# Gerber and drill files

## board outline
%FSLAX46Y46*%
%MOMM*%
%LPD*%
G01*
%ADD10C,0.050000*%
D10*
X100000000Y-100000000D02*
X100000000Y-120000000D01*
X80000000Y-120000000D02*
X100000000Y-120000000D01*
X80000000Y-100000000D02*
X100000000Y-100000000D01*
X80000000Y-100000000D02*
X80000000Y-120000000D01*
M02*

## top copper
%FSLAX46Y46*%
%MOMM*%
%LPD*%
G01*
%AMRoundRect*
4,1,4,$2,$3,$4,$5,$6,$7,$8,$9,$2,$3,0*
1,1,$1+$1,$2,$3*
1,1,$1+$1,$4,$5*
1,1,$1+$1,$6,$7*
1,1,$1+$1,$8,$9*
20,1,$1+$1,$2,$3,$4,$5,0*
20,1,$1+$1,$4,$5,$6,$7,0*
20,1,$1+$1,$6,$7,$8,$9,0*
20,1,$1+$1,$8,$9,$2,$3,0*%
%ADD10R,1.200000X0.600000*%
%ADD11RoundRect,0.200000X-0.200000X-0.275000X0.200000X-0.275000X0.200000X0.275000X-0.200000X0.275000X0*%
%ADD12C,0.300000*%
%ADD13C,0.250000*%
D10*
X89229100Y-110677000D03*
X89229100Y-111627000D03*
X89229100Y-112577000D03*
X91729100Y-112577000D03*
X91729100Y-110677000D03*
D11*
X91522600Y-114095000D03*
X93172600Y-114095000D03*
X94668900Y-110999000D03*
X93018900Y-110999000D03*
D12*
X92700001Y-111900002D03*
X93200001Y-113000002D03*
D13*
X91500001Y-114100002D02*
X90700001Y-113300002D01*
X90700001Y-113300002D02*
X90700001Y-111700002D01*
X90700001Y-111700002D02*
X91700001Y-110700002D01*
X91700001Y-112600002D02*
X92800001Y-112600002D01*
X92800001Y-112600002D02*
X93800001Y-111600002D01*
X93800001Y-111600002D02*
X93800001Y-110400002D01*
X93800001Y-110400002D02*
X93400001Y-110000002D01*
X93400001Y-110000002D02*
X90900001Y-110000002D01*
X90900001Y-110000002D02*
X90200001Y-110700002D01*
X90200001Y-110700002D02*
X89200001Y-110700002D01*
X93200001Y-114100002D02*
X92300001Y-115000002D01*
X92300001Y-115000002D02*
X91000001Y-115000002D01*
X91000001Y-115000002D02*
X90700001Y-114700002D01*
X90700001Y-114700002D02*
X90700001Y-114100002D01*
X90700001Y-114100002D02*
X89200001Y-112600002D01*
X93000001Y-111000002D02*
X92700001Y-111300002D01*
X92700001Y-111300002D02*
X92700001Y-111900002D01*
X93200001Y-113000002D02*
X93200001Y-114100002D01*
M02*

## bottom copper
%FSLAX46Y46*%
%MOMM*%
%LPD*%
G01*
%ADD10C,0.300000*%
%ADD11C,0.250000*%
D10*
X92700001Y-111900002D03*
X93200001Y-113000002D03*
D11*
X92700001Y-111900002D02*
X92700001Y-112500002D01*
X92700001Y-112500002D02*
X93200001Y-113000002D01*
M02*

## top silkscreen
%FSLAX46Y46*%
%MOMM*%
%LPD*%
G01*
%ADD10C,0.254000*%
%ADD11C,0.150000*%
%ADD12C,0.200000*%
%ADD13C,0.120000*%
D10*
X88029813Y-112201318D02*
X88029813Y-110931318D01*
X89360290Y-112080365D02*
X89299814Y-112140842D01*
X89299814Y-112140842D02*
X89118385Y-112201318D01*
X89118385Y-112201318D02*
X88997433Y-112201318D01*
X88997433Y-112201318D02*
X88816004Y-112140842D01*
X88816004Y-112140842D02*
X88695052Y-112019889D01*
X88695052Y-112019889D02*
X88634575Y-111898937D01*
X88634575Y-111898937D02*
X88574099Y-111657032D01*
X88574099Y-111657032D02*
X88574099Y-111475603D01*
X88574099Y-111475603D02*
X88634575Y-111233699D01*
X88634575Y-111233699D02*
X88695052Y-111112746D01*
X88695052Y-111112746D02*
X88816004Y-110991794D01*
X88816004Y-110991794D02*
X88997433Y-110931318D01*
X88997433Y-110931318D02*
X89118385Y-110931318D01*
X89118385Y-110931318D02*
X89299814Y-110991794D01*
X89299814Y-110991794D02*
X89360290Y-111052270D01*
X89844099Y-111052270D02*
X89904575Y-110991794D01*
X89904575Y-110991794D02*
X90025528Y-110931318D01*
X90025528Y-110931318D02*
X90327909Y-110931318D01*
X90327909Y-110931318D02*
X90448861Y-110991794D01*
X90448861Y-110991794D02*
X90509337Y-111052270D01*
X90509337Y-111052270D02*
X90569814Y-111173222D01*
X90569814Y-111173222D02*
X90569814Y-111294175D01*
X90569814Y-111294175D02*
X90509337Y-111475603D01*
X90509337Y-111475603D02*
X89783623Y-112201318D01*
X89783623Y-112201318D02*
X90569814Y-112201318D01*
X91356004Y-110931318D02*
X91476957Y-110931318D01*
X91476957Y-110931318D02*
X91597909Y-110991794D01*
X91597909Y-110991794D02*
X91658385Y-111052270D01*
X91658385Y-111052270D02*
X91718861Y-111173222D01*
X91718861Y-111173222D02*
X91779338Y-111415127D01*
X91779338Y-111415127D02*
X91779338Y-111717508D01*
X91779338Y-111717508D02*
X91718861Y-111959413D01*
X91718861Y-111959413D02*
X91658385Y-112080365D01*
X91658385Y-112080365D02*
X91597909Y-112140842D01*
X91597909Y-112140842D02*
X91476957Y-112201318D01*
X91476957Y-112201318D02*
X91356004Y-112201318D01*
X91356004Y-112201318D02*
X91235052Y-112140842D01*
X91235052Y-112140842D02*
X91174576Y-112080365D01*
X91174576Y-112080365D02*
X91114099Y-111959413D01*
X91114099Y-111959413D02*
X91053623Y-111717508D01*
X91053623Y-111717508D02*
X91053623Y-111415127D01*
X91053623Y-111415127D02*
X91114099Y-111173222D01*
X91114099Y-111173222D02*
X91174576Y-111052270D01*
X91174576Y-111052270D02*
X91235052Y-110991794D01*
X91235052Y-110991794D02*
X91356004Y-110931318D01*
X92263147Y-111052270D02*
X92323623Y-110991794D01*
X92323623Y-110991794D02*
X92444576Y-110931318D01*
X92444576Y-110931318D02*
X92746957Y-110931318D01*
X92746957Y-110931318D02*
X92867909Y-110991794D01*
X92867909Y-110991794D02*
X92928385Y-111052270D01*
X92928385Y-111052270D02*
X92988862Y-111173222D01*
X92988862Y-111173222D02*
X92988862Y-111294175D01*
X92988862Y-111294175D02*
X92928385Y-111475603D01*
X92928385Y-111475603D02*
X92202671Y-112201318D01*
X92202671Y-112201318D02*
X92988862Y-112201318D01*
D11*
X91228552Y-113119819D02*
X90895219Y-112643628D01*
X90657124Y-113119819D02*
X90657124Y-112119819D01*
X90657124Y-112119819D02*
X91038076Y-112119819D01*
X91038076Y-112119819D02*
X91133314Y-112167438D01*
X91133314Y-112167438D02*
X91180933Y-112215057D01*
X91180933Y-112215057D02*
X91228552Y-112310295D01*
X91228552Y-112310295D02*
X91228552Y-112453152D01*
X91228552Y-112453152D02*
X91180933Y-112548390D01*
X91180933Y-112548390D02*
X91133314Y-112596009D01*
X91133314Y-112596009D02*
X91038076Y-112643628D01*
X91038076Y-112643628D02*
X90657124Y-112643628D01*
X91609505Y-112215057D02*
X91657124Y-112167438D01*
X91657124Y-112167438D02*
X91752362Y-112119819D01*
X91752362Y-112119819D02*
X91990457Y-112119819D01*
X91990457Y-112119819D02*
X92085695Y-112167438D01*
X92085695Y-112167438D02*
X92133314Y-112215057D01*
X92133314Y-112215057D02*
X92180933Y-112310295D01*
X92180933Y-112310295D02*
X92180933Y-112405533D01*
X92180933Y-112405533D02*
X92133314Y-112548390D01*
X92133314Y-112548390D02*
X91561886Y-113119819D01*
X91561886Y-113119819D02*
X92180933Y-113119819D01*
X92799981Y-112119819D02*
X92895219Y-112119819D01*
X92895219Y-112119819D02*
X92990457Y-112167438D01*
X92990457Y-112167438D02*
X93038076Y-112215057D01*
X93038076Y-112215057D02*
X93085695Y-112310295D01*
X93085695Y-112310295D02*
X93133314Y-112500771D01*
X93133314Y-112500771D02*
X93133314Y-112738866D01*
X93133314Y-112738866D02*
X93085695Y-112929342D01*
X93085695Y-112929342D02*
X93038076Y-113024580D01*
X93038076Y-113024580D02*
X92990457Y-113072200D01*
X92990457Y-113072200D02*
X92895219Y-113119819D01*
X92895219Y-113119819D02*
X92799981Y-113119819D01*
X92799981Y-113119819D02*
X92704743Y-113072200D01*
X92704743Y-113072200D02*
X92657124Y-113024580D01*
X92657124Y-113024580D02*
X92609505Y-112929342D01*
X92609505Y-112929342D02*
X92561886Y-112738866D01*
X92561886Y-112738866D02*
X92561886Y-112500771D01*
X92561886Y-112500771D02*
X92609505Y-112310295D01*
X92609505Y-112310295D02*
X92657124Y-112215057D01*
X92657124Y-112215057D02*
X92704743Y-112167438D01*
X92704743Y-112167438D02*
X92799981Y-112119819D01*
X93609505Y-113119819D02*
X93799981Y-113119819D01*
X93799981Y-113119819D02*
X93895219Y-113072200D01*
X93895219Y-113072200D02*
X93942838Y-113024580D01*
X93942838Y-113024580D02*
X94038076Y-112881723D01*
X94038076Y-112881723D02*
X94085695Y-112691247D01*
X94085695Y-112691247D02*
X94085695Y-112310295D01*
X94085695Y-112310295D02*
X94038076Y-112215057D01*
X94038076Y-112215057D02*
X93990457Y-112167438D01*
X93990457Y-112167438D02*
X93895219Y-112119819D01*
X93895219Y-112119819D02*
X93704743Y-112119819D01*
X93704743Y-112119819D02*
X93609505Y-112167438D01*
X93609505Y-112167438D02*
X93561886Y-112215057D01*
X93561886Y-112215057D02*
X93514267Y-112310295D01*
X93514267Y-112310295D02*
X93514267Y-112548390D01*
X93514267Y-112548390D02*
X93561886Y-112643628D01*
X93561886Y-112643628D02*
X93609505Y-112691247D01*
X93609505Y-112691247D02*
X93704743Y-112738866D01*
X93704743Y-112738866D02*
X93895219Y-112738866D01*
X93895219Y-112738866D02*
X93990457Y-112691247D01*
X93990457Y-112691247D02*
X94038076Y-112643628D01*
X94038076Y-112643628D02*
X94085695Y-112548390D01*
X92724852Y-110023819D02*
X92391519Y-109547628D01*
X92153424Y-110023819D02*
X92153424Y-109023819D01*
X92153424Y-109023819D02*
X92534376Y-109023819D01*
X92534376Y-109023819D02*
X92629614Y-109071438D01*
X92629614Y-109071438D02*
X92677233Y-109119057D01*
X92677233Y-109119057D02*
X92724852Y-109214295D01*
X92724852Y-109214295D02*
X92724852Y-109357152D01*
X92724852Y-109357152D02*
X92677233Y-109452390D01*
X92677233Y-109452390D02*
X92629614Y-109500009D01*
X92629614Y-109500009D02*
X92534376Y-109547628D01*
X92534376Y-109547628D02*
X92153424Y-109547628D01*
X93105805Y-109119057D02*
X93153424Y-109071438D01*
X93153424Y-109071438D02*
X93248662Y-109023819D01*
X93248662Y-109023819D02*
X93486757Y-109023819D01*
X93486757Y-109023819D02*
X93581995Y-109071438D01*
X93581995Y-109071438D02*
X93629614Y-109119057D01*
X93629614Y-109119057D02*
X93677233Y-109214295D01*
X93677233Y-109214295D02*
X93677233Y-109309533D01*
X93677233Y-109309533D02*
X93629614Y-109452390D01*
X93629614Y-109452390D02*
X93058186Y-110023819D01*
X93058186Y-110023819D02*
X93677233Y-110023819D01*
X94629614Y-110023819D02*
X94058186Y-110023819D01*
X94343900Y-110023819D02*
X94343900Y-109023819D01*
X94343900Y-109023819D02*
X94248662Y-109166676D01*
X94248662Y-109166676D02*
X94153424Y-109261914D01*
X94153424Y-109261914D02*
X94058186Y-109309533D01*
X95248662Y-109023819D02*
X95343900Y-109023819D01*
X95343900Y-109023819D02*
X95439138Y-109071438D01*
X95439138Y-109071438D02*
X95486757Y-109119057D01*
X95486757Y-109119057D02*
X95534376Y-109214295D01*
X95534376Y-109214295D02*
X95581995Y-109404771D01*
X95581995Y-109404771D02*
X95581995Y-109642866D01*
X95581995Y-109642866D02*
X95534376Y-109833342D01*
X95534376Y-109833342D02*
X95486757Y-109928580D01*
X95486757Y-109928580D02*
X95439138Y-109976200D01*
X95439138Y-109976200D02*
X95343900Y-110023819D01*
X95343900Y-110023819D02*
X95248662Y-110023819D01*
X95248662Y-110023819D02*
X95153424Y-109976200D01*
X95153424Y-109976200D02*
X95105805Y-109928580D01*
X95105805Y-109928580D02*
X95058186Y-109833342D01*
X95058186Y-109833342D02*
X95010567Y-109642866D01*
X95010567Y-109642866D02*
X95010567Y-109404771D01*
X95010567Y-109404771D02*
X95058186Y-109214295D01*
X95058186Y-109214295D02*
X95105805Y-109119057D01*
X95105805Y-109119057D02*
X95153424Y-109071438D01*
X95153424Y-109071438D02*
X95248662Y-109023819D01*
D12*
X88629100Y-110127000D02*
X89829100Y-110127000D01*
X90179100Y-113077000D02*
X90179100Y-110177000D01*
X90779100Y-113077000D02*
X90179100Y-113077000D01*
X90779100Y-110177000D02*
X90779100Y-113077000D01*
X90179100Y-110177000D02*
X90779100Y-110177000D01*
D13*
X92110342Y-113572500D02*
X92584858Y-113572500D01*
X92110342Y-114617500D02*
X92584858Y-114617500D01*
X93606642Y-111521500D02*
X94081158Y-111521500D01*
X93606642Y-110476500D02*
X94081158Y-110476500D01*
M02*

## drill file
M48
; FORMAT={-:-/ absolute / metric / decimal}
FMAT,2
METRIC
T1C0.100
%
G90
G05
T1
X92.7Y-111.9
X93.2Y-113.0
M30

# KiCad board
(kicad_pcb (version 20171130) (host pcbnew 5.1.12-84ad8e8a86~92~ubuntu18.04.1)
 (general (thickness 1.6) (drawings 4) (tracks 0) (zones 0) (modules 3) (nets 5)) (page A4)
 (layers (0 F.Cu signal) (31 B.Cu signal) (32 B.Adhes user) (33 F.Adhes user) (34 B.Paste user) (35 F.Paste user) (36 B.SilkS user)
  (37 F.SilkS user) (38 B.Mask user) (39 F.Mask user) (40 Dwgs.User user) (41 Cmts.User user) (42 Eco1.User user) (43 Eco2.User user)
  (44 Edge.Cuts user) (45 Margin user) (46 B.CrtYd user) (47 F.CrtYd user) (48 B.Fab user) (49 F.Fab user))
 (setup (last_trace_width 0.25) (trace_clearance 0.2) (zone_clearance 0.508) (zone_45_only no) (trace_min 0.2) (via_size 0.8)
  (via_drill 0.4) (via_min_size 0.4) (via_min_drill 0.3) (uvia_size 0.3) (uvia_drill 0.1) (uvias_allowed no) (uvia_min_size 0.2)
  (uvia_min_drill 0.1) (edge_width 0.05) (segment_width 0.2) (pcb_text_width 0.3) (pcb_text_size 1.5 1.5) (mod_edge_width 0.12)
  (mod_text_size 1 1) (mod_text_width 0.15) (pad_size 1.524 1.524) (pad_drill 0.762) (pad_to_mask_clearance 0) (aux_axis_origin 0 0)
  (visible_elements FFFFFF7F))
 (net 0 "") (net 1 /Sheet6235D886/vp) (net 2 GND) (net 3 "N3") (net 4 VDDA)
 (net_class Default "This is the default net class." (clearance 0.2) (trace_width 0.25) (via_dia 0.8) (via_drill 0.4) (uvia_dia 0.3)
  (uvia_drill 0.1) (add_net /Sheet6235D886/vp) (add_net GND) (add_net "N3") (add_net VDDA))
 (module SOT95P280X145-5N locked (layer F.Cu) (at 90.479100 111.627000)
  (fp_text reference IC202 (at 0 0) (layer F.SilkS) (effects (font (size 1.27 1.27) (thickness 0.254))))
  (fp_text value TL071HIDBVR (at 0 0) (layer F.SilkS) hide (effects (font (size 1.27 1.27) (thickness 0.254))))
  (fp_line (start -1.85 -1.5) (end -0.65 -1.5) (layer F.SilkS) (width 0.2))
  (fp_line (start -0.3 1.45) (end -0.3 -1.45) (layer F.SilkS) (width 0.2))
  (fp_line (start 0.3 1.45) (end -0.3 1.45) (layer F.SilkS) (width 0.2))
  (fp_line (start 0.3 -1.45) (end 0.3 1.45) (layer F.SilkS) (width 0.2))
  (fp_line (start -0.3 -1.45) (end 0.3 -1.45) (layer F.SilkS) (width 0.2))
  (pad 1 smd rect (at -1.25 -0.95 90.000000) (size 0.6 1.2) (layers F.Cu F.Mask F.Paste) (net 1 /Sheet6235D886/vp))
  (pad 2 smd rect (at -1.25 0 90.000000) (size 0.6 1.2) (layers F.Cu F.Mask F.Paste) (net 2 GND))
  (pad 3 smd rect (at -1.25 0.95 90.000000) (size 0.6 1.2) (layers F.Cu F.Mask F.Paste) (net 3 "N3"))
  (pad 4 smd rect (at 1.25 0.95 90.000000) (size 0.6 1.2) (layers F.Cu F.Mask F.Paste) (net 1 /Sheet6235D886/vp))
  (pad 5 smd rect (at 1.25 -0.95 90.000000) (size 0.6 1.2) (layers F.Cu F.Mask F.Paste) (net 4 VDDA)))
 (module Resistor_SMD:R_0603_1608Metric (layer F.Cu) (at 92.347600 114.095000)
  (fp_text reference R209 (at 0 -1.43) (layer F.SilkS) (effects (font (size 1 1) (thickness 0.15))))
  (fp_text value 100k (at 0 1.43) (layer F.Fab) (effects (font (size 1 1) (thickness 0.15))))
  (fp_line (start -0.237258 -0.5225) (end 0.237258 -0.5225) (layer F.SilkS) (width 0.12))
  (fp_line (start -0.237258 0.5225) (end 0.237258 0.5225) (layer F.SilkS) (width 0.12))
  (pad 1 smd roundrect (at -0.825 0) (size 0.8 0.95) (layers F.Cu F.Mask F.Paste) (roundrect_rratio 0.25) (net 4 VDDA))
  (pad 2 smd roundrect (at 0.825 0) (size 0.8 0.95) (layers F.Cu F.Mask F.Paste) (roundrect_rratio 0.25) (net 3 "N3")))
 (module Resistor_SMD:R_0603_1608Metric (layer F.Cu) (at 93.843900 110.999000)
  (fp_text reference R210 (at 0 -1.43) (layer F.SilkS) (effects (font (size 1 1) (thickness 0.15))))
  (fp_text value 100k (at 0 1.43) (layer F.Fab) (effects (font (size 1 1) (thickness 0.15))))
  (fp_line (start -0.237258 0.5225) (end 0.237258 0.5225) (layer F.SilkS) (width 0.12))
  (fp_line (start -0.237258 -0.5225) (end 0.237258 -0.5225) (layer F.SilkS) (width 0.12))
  (pad 2 smd roundrect (at 0.825 0) (size 0.8 0.95) (layers F.Cu F.Mask F.Paste) (roundrect_rratio 0.25) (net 2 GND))
  (pad 1 smd roundrect (at -0.825 0) (size 0.8 0.95) (layers F.Cu F.Mask F.Paste) (roundrect_rratio 0.25) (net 3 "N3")))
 (gr_line (start 100 100) (end 100 120) (layer Edge.Cuts) (width 0.05))
 (gr_line (start 80 120) (end 100 120) (layer Edge.Cuts) (width 0.05))
 (gr_line (start 80 100) (end 100 100) (layer Edge.Cuts) (width 0.05))
 (gr_line (start 80 100) (end 80 120) (layer Edge.Cuts) (width 0.05))
 (segment (start 91.500001 114.100002) (end 90.700001 113.300002) (width 0.250000) (layer F.Cu) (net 4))
 (segment (start 90.700001 113.300002) (end 90.700001 111.700002) (width 0.250000) (layer F.Cu) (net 4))
 (segment (start 90.700001 111.700002) (end 91.700001 110.700002) (width 0.250000) (layer F.Cu) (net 4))
 (segment (start 91.700001 112.600002) (end 92.800001 112.600002) (width 0.250000) (layer F.Cu) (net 1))
 (segment (start 92.800001 112.600002) (end 93.800001 111.600002) (width 0.250000) (layer F.Cu) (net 1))
 (segment (start 93.800001 111.600002) (end 93.800001 110.400002) (width 0.250000) (layer F.Cu) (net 1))
 (segment (start 93.800001 110.400002) (end 93.400001 110.000002) (width 0.250000) (layer F.Cu) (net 1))
 (segment (start 93.400001 110.000002) (end 90.900001 110.000002) (width 0.250000) (layer F.Cu) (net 1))
 (segment (start 90.900001 110.000002) (end 90.200001 110.700002) (width 0.250000) (layer F.Cu) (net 1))
 (segment (start 90.200001 110.700002) (end 89.200001 110.700002) (width 0.250000) (layer F.Cu) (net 1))
 (segment (start 93.200001 114.100002) (end 92.300001 115.000002) (width 0.250000) (layer F.Cu) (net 3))
 (segment (start 92.300001 115.000002) (end 91.000001 115.000002) (width 0.250000) (layer F.Cu) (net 3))
 (segment (start 91.000001 115.000002) (end 90.700001 114.700002) (width 0.250000) (layer F.Cu) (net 3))
 (segment (start 90.700001 114.700002) (end 90.700001 114.100002) (width 0.250000) (layer F.Cu) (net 3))
 (segment (start 90.700001 114.100002) (end 89.200001 112.600002) (width 0.250000) (layer F.Cu) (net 3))
 (segment (start 93.000001 111.000002) (end 92.700001 111.300002) (width 0.250000) (layer F.Cu) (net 3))
 (segment (start 92.700001 111.300002) (end 92.700001 111.900002) (width 0.250000) (layer F.Cu) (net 3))
 (segment (start 92.700001 111.900002) (end 92.700001 112.500002) (width 0.250000) (layer B.Cu) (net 3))
 (segment (start 92.700001 112.500002) (end 93.200001 113.000002) (width 0.250000) (layer B.Cu) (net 3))
 (segment (start 93.200001 113.000002) (end 93.200001 114.100002) (width 0.250000) (layer F.Cu) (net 3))
 (via micro (at 92.700001 111.900002) (size 0.300000) (drill 0.100000) (layers F.Cu B.Cu) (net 3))
 (via micro (at 93.200001 113.000002) (size 0.300000) (drill 0.100000) (layers F.Cu B.Cu) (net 3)))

